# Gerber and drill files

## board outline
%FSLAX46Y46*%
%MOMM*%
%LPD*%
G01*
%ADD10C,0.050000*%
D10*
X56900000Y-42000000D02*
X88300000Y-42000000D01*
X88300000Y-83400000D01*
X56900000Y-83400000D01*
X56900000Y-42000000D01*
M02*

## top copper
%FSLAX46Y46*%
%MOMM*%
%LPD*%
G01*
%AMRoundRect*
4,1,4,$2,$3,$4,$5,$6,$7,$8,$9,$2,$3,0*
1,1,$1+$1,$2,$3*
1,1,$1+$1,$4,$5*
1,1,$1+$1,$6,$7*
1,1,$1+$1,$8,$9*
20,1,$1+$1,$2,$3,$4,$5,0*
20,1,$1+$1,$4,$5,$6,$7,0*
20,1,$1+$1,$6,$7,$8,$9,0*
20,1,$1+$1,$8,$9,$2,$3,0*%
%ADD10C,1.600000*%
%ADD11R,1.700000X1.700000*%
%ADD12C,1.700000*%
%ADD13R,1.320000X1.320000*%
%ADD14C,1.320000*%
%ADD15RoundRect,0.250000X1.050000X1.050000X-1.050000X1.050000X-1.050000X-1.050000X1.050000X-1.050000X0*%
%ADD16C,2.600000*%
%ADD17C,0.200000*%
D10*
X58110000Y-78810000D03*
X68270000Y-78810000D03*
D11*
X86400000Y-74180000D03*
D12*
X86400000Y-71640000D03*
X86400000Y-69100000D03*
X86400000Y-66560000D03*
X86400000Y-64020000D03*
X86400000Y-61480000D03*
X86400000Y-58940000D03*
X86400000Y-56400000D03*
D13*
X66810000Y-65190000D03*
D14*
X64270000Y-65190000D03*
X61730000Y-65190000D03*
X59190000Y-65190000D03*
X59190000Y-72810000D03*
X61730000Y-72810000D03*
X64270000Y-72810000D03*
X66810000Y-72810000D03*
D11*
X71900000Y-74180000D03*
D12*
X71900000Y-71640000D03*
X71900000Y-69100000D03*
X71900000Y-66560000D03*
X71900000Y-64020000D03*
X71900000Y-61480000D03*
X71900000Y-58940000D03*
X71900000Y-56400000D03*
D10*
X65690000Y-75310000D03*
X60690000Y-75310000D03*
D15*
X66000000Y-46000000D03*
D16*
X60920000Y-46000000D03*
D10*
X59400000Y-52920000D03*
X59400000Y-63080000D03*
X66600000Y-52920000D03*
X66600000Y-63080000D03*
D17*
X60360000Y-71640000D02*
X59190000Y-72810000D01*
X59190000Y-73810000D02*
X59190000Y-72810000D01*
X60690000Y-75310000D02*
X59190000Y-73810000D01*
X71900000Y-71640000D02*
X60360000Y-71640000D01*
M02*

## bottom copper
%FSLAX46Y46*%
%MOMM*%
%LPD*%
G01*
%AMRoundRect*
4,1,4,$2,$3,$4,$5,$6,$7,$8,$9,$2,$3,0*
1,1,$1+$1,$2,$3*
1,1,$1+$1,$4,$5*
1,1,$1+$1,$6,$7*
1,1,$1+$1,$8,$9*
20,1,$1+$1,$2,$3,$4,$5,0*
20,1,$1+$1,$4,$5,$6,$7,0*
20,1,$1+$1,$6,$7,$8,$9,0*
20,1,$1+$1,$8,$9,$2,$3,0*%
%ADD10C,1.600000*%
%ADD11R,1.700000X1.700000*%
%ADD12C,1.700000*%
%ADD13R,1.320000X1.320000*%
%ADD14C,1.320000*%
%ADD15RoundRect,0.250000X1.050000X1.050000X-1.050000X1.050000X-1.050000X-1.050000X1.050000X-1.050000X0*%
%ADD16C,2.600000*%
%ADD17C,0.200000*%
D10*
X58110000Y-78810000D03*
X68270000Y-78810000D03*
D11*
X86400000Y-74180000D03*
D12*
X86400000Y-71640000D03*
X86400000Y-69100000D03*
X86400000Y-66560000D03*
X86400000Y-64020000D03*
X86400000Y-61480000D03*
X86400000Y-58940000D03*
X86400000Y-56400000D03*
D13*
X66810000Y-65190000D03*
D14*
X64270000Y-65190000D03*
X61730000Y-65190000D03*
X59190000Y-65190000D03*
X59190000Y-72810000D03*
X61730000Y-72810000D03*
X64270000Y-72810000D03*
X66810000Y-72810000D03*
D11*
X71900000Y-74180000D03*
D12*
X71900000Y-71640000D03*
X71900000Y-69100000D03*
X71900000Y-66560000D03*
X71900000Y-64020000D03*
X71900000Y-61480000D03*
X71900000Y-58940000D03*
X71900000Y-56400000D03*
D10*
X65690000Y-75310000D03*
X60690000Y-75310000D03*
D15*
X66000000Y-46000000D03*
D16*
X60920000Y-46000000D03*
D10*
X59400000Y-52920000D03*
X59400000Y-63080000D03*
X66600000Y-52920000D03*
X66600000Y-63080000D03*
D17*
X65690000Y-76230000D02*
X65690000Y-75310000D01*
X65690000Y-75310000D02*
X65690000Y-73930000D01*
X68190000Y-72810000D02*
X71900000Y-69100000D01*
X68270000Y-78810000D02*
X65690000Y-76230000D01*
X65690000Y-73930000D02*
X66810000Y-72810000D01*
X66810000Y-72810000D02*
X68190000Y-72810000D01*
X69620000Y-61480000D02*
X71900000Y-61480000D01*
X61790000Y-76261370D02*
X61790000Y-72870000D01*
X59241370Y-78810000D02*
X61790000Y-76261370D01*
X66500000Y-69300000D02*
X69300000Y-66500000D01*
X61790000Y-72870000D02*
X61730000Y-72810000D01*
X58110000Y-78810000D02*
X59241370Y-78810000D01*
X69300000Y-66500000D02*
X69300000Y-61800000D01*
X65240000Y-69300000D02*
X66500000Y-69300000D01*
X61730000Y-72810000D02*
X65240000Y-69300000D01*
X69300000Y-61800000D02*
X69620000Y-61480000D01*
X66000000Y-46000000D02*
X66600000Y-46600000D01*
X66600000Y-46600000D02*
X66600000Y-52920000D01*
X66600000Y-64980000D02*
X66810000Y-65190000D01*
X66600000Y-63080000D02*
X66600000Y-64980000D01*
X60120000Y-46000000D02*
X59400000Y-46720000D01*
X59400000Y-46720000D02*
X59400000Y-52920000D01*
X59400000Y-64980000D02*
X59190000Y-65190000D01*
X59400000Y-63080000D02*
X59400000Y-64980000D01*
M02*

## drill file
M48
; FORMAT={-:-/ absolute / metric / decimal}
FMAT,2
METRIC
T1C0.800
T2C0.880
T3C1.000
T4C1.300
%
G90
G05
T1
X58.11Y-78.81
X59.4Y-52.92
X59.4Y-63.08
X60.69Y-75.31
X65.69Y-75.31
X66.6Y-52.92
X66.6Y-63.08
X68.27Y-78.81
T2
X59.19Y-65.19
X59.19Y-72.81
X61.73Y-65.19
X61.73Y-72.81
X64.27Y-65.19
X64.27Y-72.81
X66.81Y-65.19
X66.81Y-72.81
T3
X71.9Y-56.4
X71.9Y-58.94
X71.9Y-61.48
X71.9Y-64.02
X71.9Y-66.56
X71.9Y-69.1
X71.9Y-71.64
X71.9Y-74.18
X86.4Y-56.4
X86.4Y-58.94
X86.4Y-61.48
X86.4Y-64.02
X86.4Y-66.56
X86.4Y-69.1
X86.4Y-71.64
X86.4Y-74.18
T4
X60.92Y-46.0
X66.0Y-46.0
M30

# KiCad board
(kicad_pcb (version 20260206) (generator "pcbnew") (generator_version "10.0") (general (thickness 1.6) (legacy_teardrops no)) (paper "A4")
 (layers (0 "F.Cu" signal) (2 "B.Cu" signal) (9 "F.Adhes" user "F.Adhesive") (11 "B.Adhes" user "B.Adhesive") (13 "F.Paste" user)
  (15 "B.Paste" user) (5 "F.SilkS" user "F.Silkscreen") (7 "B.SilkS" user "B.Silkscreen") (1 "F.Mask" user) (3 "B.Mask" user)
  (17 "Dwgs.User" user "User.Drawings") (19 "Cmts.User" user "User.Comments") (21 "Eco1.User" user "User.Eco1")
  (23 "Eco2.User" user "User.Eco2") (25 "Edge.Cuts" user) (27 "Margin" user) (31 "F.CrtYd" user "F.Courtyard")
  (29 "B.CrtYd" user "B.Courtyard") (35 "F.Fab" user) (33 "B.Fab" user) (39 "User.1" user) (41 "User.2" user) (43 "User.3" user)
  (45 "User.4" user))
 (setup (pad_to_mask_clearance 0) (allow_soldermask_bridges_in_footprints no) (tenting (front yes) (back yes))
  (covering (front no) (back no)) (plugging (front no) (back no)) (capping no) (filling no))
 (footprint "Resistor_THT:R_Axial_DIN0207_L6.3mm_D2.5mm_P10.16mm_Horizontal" (layer "F.Cu") (at 58.11 78.81)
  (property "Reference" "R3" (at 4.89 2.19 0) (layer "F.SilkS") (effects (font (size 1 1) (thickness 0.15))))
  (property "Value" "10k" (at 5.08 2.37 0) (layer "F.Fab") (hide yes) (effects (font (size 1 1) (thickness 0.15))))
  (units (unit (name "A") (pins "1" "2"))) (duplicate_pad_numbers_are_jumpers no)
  (pad "1" thru_hole circle (at 0 0) (size 1.6 1.6) (drill 0.8) (layers "*.Cu" "*.Mask") (remove_unused_layers no) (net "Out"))
  (pad "2" thru_hole circle (at 10.16 0) (size 1.6 1.6) (drill 0.8) (layers "*.Cu" "*.Mask") (remove_unused_layers no) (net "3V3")))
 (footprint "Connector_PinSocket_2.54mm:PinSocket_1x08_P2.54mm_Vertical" (layer "F.Cu") (at 86.4 74.18 180)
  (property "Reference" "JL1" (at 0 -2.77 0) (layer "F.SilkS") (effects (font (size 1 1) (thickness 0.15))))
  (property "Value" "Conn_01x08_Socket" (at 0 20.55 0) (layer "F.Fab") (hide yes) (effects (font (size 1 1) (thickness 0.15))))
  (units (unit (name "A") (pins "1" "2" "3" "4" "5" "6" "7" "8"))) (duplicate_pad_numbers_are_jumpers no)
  (pad "1" thru_hole rect (at 0 0 180) (size 1.7 1.7) (drill 1) (layers "*.Cu" "*.Mask") (remove_unused_layers no)
   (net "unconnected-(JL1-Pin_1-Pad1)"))
  (pad "2" thru_hole circle (at 0 2.54 180) (size 1.7 1.7) (drill 1) (layers "*.Cu" "*.Mask") (remove_unused_layers no)
   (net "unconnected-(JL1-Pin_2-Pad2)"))
  (pad "3" thru_hole circle (at 0 5.08 180) (size 1.7 1.7) (drill 1) (layers "*.Cu" "*.Mask") (remove_unused_layers no)
   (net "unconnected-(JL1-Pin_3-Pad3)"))
  (pad "4" thru_hole circle (at 0 7.62 180) (size 1.7 1.7) (drill 1) (layers "*.Cu" "*.Mask") (remove_unused_layers no)
   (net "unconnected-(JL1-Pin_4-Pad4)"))
  (pad "5" thru_hole circle (at 0 10.16 180) (size 1.7 1.7) (drill 1) (layers "*.Cu" "*.Mask") (remove_unused_layers no)
   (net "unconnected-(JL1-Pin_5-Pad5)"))
  (pad "6" thru_hole circle (at 0 12.7 180) (size 1.7 1.7) (drill 1) (layers "*.Cu" "*.Mask") (remove_unused_layers no)
   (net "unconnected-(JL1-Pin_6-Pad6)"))
  (pad "7" thru_hole circle (at 0 15.24 180) (size 1.7 1.7) (drill 1) (layers "*.Cu" "*.Mask") (remove_unused_layers no)
   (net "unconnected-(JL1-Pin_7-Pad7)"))
  (pad "8" thru_hole circle (at 0 17.78 180) (size 1.7 1.7) (drill 1) (layers "*.Cu" "*.Mask") (remove_unused_layers no)
   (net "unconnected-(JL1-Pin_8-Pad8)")))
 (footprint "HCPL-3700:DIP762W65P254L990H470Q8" (layer "F.Cu") (at 63 69 -90)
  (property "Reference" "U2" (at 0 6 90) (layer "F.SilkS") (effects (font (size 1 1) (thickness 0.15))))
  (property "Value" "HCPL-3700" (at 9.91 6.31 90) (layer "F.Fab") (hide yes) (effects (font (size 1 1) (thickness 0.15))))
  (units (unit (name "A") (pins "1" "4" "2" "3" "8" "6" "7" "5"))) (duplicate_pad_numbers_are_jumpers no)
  (pad "1" thru_hole rect (at -3.81 -3.81 270) (size 1.32 1.32) (drill 0.88) (layers "*.Cu" "*.Mask") (remove_unused_layers no)
   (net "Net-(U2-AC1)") (solder_mask_margin 0.102))
  (pad "2" thru_hole circle (at -3.81 -1.27 270) (size 1.32 1.32) (drill 0.88) (layers "*.Cu" "*.Mask") (remove_unused_layers no)
   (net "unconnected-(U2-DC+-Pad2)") (solder_mask_margin 0.102))
  (pad "3" thru_hole circle (at -3.81 1.27 270) (size 1.32 1.32) (drill 0.88) (layers "*.Cu" "*.Mask") (remove_unused_layers no)
   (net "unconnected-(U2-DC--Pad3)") (solder_mask_margin 0.102))
  (pad "4" thru_hole circle (at -3.81 3.81 270) (size 1.32 1.32) (drill 0.88) (layers "*.Cu" "*.Mask") (remove_unused_layers no)
   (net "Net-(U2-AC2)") (solder_mask_margin 0.102))
  (pad "5" thru_hole circle (at 3.81 3.81 270) (size 1.32 1.32) (drill 0.88) (layers "*.Cu" "*.Mask") (remove_unused_layers no) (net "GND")
   (solder_mask_margin 0.102))
  (pad "6" thru_hole circle (at 3.81 1.27 270) (size 1.32 1.32) (drill 0.88) (layers "*.Cu" "*.Mask") (remove_unused_layers no) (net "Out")
   (solder_mask_margin 0.102))
  (pad "7" thru_hole circle (at 3.81 -1.27 270) (size 1.32 1.32) (drill 0.88) (layers "*.Cu" "*.Mask") (remove_unused_layers no)
   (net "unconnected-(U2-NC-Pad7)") (solder_mask_margin 0.102))
  (pad "8" thru_hole circle (at 3.81 -3.81 270) (size 1.32 1.32) (drill 0.88) (layers "*.Cu" "*.Mask") (remove_unused_layers no) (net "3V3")
   (solder_mask_margin 0.102)))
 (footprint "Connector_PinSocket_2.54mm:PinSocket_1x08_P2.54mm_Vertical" (layer "F.Cu") (at 71.9 74.18 180)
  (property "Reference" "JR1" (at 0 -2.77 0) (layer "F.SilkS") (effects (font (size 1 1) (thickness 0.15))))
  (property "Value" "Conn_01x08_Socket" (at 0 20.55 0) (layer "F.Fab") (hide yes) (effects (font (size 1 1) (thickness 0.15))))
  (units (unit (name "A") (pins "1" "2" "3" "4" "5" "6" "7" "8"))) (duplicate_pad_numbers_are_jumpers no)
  (pad "1" thru_hole rect (at 0 0 180) (size 1.7 1.7) (drill 1) (layers "*.Cu" "*.Mask") (remove_unused_layers no)
   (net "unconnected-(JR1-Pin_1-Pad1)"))
  (pad "2" thru_hole circle (at 0 2.54 180) (size 1.7 1.7) (drill 1) (layers "*.Cu" "*.Mask") (remove_unused_layers no) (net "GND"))
  (pad "3" thru_hole circle (at 0 5.08 180) (size 1.7 1.7) (drill 1) (layers "*.Cu" "*.Mask") (remove_unused_layers no) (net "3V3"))
  (pad "4" thru_hole circle (at 0 7.62 180) (size 1.7 1.7) (drill 1) (layers "*.Cu" "*.Mask") (remove_unused_layers no)
   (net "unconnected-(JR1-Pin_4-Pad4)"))
  (pad "5" thru_hole circle (at 0 10.16 180) (size 1.7 1.7) (drill 1) (layers "*.Cu" "*.Mask") (remove_unused_layers no)
   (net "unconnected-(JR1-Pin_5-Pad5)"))
  (pad "6" thru_hole circle (at 0 12.7 180) (size 1.7 1.7) (drill 1) (layers "*.Cu" "*.Mask") (remove_unused_layers no) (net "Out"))
  (pad "7" thru_hole circle (at 0 15.24 180) (size 1.7 1.7) (drill 1) (layers "*.Cu" "*.Mask") (remove_unused_layers no)
   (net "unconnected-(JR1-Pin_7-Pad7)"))
  (pad "8" thru_hole circle (at 0 17.78 180) (size 1.7 1.7) (drill 1) (layers "*.Cu" "*.Mask") (remove_unused_layers no)
   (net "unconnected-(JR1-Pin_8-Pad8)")))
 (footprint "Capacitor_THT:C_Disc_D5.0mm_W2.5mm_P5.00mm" (layer "F.Cu") (at 65.69 75.31 180)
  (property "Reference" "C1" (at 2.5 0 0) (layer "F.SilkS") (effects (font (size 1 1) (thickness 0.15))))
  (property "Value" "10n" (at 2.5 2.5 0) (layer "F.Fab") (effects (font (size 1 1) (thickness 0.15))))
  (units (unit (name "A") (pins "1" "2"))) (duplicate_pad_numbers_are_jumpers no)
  (pad "1" thru_hole circle (at 0 0 180) (size 1.6 1.6) (drill 0.8) (layers "*.Cu" "*.Mask") (remove_unused_layers no) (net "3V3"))
  (pad "2" thru_hole circle (at 5 0 180) (size 1.6 1.6) (drill 0.8) (layers "*.Cu" "*.Mask") (remove_unused_layers no) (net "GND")))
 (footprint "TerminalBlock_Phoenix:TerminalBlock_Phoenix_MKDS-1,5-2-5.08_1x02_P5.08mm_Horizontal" (layer "F.Cu") (at 66 46 180)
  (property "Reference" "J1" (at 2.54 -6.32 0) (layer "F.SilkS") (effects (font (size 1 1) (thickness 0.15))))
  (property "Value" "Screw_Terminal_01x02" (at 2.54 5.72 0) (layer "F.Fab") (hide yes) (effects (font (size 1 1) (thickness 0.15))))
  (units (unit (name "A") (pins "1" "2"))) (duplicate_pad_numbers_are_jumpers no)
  (pad "1" thru_hole roundrect (at 0 0 180) (size 2.6 2.6) (drill 1.3) (layers "*.Cu" "*.Mask") (remove_unused_layers no)
   (roundrect_rratio 0.096154) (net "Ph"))
  (pad "2" thru_hole circle (at 5.08 0 180) (size 2.6 2.6) (drill 1.3) (layers "*.Cu" "*.Mask") (remove_unused_layers no) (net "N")))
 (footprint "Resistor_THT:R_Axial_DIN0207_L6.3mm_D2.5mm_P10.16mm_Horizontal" (layer "F.Cu") (at 59.4 52.92 -90)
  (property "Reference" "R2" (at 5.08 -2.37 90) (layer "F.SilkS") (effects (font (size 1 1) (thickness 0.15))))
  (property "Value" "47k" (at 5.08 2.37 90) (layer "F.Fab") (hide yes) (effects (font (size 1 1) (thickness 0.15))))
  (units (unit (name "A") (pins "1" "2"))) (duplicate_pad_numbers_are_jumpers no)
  (pad "1" thru_hole circle (at 0 0 270) (size 1.6 1.6) (drill 0.8) (layers "*.Cu" "*.Mask") (remove_unused_layers no) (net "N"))
  (pad "2" thru_hole circle (at 10.16 0 270) (size 1.6 1.6) (drill 0.8) (layers "*.Cu" "*.Mask") (remove_unused_layers no)
   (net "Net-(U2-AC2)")))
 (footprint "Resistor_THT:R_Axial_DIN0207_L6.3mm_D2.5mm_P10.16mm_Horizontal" (layer "F.Cu") (at 66.6 52.92 -90)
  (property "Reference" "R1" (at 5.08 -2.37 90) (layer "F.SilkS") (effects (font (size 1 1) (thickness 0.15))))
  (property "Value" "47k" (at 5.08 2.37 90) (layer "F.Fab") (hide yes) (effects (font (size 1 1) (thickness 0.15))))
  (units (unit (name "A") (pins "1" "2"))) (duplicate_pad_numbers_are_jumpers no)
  (pad "1" thru_hole circle (at 0 0 270) (size 1.6 1.6) (drill 0.8) (layers "*.Cu" "*.Mask") (remove_unused_layers no) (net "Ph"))
  (pad "2" thru_hole circle (at 10.16 0 270) (size 1.6 1.6) (drill 0.8) (layers "*.Cu" "*.Mask") (remove_unused_layers no)
   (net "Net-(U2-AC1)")))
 (gr_rect (start 56.9 42) (end 88.3 83.4) (stroke (width 0.05) (type default)) (fill no) (layer "Edge.Cuts"))
 (segment (start 65.69 76.23) (end 65.69 75.31) (width 0.2) (layer "B.Cu") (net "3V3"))
 (segment (start 65.69 75.31) (end 65.69 73.93) (width 0.2) (layer "B.Cu") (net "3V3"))
 (segment (start 68.19 72.81) (end 71.9 69.1) (width 0.2) (layer "B.Cu") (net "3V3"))
 (segment (start 68.27 78.81) (end 65.69 76.23) (width 0.2) (layer "B.Cu") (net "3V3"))
 (segment (start 65.69 73.93) (end 66.81 72.81) (width 0.2) (layer "B.Cu") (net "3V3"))
 (segment (start 66.81 72.81) (end 68.19 72.81) (width 0.2) (layer "B.Cu") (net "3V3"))
 (segment (start 60.36 71.64) (end 59.19 72.81) (width 0.2) (layer "F.Cu") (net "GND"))
 (segment (start 59.19 73.81) (end 59.19 72.81) (width 0.2) (layer "F.Cu") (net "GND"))
 (segment (start 60.69 75.31) (end 59.19 73.81) (width 0.2) (layer "F.Cu") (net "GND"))
 (segment (start 71.9 71.64) (end 60.36 71.64) (width 0.2) (layer "F.Cu") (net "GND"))
 (segment (start 69.62 61.48) (end 71.9 61.48) (width 0.2) (layer "B.Cu") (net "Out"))
 (segment (start 61.79 76.26137) (end 61.79 72.87) (width 0.2) (layer "B.Cu") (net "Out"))
 (segment (start 59.24137 78.81) (end 61.79 76.26137) (width 0.2) (layer "B.Cu") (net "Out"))
 (segment (start 66.5 69.3) (end 69.3 66.5) (width 0.2) (layer "B.Cu") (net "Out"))
 (segment (start 61.79 72.87) (end 61.73 72.81) (width 0.2) (layer "B.Cu") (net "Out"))
 (segment (start 58.11 78.81) (end 59.24137 78.81) (width 0.2) (layer "B.Cu") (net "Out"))
 (segment (start 69.3 66.5) (end 69.3 61.8) (width 0.2) (layer "B.Cu") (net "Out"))
 (segment (start 65.24 69.3) (end 66.5 69.3) (width 0.2) (layer "B.Cu") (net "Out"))
 (segment (start 61.73 72.81) (end 65.24 69.3) (width 0.2) (layer "B.Cu") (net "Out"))
 (segment (start 69.3 61.8) (end 69.62 61.48) (width 0.2) (layer "B.Cu") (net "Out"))
 (segment (start 66 46) (end 66.6 46.6) (width 0.2) (layer "B.Cu") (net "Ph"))
 (segment (start 66.6 46.6) (end 66.6 52.92) (width 0.2) (layer "B.Cu") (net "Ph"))
 (segment (start 66.6 64.98) (end 66.81 65.19) (width 0.2) (layer "B.Cu") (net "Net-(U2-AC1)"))
 (segment (start 66.6 63.08) (end 66.6 64.98) (width 0.2) (layer "B.Cu") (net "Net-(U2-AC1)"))
 (segment (start 60.12 46) (end 59.4 46.72) (width 0.2) (layer "B.Cu") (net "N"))
 (segment (start 59.4 46.72) (end 59.4 52.92) (width 0.2) (layer "B.Cu") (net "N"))
 (segment (start 59.4 64.98) (end 59.19 65.19) (width 0.2) (layer "B.Cu") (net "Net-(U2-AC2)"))
 (segment (start 59.4 63.08) (end 59.4 64.98) (width 0.2) (layer "B.Cu") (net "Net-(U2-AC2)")))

